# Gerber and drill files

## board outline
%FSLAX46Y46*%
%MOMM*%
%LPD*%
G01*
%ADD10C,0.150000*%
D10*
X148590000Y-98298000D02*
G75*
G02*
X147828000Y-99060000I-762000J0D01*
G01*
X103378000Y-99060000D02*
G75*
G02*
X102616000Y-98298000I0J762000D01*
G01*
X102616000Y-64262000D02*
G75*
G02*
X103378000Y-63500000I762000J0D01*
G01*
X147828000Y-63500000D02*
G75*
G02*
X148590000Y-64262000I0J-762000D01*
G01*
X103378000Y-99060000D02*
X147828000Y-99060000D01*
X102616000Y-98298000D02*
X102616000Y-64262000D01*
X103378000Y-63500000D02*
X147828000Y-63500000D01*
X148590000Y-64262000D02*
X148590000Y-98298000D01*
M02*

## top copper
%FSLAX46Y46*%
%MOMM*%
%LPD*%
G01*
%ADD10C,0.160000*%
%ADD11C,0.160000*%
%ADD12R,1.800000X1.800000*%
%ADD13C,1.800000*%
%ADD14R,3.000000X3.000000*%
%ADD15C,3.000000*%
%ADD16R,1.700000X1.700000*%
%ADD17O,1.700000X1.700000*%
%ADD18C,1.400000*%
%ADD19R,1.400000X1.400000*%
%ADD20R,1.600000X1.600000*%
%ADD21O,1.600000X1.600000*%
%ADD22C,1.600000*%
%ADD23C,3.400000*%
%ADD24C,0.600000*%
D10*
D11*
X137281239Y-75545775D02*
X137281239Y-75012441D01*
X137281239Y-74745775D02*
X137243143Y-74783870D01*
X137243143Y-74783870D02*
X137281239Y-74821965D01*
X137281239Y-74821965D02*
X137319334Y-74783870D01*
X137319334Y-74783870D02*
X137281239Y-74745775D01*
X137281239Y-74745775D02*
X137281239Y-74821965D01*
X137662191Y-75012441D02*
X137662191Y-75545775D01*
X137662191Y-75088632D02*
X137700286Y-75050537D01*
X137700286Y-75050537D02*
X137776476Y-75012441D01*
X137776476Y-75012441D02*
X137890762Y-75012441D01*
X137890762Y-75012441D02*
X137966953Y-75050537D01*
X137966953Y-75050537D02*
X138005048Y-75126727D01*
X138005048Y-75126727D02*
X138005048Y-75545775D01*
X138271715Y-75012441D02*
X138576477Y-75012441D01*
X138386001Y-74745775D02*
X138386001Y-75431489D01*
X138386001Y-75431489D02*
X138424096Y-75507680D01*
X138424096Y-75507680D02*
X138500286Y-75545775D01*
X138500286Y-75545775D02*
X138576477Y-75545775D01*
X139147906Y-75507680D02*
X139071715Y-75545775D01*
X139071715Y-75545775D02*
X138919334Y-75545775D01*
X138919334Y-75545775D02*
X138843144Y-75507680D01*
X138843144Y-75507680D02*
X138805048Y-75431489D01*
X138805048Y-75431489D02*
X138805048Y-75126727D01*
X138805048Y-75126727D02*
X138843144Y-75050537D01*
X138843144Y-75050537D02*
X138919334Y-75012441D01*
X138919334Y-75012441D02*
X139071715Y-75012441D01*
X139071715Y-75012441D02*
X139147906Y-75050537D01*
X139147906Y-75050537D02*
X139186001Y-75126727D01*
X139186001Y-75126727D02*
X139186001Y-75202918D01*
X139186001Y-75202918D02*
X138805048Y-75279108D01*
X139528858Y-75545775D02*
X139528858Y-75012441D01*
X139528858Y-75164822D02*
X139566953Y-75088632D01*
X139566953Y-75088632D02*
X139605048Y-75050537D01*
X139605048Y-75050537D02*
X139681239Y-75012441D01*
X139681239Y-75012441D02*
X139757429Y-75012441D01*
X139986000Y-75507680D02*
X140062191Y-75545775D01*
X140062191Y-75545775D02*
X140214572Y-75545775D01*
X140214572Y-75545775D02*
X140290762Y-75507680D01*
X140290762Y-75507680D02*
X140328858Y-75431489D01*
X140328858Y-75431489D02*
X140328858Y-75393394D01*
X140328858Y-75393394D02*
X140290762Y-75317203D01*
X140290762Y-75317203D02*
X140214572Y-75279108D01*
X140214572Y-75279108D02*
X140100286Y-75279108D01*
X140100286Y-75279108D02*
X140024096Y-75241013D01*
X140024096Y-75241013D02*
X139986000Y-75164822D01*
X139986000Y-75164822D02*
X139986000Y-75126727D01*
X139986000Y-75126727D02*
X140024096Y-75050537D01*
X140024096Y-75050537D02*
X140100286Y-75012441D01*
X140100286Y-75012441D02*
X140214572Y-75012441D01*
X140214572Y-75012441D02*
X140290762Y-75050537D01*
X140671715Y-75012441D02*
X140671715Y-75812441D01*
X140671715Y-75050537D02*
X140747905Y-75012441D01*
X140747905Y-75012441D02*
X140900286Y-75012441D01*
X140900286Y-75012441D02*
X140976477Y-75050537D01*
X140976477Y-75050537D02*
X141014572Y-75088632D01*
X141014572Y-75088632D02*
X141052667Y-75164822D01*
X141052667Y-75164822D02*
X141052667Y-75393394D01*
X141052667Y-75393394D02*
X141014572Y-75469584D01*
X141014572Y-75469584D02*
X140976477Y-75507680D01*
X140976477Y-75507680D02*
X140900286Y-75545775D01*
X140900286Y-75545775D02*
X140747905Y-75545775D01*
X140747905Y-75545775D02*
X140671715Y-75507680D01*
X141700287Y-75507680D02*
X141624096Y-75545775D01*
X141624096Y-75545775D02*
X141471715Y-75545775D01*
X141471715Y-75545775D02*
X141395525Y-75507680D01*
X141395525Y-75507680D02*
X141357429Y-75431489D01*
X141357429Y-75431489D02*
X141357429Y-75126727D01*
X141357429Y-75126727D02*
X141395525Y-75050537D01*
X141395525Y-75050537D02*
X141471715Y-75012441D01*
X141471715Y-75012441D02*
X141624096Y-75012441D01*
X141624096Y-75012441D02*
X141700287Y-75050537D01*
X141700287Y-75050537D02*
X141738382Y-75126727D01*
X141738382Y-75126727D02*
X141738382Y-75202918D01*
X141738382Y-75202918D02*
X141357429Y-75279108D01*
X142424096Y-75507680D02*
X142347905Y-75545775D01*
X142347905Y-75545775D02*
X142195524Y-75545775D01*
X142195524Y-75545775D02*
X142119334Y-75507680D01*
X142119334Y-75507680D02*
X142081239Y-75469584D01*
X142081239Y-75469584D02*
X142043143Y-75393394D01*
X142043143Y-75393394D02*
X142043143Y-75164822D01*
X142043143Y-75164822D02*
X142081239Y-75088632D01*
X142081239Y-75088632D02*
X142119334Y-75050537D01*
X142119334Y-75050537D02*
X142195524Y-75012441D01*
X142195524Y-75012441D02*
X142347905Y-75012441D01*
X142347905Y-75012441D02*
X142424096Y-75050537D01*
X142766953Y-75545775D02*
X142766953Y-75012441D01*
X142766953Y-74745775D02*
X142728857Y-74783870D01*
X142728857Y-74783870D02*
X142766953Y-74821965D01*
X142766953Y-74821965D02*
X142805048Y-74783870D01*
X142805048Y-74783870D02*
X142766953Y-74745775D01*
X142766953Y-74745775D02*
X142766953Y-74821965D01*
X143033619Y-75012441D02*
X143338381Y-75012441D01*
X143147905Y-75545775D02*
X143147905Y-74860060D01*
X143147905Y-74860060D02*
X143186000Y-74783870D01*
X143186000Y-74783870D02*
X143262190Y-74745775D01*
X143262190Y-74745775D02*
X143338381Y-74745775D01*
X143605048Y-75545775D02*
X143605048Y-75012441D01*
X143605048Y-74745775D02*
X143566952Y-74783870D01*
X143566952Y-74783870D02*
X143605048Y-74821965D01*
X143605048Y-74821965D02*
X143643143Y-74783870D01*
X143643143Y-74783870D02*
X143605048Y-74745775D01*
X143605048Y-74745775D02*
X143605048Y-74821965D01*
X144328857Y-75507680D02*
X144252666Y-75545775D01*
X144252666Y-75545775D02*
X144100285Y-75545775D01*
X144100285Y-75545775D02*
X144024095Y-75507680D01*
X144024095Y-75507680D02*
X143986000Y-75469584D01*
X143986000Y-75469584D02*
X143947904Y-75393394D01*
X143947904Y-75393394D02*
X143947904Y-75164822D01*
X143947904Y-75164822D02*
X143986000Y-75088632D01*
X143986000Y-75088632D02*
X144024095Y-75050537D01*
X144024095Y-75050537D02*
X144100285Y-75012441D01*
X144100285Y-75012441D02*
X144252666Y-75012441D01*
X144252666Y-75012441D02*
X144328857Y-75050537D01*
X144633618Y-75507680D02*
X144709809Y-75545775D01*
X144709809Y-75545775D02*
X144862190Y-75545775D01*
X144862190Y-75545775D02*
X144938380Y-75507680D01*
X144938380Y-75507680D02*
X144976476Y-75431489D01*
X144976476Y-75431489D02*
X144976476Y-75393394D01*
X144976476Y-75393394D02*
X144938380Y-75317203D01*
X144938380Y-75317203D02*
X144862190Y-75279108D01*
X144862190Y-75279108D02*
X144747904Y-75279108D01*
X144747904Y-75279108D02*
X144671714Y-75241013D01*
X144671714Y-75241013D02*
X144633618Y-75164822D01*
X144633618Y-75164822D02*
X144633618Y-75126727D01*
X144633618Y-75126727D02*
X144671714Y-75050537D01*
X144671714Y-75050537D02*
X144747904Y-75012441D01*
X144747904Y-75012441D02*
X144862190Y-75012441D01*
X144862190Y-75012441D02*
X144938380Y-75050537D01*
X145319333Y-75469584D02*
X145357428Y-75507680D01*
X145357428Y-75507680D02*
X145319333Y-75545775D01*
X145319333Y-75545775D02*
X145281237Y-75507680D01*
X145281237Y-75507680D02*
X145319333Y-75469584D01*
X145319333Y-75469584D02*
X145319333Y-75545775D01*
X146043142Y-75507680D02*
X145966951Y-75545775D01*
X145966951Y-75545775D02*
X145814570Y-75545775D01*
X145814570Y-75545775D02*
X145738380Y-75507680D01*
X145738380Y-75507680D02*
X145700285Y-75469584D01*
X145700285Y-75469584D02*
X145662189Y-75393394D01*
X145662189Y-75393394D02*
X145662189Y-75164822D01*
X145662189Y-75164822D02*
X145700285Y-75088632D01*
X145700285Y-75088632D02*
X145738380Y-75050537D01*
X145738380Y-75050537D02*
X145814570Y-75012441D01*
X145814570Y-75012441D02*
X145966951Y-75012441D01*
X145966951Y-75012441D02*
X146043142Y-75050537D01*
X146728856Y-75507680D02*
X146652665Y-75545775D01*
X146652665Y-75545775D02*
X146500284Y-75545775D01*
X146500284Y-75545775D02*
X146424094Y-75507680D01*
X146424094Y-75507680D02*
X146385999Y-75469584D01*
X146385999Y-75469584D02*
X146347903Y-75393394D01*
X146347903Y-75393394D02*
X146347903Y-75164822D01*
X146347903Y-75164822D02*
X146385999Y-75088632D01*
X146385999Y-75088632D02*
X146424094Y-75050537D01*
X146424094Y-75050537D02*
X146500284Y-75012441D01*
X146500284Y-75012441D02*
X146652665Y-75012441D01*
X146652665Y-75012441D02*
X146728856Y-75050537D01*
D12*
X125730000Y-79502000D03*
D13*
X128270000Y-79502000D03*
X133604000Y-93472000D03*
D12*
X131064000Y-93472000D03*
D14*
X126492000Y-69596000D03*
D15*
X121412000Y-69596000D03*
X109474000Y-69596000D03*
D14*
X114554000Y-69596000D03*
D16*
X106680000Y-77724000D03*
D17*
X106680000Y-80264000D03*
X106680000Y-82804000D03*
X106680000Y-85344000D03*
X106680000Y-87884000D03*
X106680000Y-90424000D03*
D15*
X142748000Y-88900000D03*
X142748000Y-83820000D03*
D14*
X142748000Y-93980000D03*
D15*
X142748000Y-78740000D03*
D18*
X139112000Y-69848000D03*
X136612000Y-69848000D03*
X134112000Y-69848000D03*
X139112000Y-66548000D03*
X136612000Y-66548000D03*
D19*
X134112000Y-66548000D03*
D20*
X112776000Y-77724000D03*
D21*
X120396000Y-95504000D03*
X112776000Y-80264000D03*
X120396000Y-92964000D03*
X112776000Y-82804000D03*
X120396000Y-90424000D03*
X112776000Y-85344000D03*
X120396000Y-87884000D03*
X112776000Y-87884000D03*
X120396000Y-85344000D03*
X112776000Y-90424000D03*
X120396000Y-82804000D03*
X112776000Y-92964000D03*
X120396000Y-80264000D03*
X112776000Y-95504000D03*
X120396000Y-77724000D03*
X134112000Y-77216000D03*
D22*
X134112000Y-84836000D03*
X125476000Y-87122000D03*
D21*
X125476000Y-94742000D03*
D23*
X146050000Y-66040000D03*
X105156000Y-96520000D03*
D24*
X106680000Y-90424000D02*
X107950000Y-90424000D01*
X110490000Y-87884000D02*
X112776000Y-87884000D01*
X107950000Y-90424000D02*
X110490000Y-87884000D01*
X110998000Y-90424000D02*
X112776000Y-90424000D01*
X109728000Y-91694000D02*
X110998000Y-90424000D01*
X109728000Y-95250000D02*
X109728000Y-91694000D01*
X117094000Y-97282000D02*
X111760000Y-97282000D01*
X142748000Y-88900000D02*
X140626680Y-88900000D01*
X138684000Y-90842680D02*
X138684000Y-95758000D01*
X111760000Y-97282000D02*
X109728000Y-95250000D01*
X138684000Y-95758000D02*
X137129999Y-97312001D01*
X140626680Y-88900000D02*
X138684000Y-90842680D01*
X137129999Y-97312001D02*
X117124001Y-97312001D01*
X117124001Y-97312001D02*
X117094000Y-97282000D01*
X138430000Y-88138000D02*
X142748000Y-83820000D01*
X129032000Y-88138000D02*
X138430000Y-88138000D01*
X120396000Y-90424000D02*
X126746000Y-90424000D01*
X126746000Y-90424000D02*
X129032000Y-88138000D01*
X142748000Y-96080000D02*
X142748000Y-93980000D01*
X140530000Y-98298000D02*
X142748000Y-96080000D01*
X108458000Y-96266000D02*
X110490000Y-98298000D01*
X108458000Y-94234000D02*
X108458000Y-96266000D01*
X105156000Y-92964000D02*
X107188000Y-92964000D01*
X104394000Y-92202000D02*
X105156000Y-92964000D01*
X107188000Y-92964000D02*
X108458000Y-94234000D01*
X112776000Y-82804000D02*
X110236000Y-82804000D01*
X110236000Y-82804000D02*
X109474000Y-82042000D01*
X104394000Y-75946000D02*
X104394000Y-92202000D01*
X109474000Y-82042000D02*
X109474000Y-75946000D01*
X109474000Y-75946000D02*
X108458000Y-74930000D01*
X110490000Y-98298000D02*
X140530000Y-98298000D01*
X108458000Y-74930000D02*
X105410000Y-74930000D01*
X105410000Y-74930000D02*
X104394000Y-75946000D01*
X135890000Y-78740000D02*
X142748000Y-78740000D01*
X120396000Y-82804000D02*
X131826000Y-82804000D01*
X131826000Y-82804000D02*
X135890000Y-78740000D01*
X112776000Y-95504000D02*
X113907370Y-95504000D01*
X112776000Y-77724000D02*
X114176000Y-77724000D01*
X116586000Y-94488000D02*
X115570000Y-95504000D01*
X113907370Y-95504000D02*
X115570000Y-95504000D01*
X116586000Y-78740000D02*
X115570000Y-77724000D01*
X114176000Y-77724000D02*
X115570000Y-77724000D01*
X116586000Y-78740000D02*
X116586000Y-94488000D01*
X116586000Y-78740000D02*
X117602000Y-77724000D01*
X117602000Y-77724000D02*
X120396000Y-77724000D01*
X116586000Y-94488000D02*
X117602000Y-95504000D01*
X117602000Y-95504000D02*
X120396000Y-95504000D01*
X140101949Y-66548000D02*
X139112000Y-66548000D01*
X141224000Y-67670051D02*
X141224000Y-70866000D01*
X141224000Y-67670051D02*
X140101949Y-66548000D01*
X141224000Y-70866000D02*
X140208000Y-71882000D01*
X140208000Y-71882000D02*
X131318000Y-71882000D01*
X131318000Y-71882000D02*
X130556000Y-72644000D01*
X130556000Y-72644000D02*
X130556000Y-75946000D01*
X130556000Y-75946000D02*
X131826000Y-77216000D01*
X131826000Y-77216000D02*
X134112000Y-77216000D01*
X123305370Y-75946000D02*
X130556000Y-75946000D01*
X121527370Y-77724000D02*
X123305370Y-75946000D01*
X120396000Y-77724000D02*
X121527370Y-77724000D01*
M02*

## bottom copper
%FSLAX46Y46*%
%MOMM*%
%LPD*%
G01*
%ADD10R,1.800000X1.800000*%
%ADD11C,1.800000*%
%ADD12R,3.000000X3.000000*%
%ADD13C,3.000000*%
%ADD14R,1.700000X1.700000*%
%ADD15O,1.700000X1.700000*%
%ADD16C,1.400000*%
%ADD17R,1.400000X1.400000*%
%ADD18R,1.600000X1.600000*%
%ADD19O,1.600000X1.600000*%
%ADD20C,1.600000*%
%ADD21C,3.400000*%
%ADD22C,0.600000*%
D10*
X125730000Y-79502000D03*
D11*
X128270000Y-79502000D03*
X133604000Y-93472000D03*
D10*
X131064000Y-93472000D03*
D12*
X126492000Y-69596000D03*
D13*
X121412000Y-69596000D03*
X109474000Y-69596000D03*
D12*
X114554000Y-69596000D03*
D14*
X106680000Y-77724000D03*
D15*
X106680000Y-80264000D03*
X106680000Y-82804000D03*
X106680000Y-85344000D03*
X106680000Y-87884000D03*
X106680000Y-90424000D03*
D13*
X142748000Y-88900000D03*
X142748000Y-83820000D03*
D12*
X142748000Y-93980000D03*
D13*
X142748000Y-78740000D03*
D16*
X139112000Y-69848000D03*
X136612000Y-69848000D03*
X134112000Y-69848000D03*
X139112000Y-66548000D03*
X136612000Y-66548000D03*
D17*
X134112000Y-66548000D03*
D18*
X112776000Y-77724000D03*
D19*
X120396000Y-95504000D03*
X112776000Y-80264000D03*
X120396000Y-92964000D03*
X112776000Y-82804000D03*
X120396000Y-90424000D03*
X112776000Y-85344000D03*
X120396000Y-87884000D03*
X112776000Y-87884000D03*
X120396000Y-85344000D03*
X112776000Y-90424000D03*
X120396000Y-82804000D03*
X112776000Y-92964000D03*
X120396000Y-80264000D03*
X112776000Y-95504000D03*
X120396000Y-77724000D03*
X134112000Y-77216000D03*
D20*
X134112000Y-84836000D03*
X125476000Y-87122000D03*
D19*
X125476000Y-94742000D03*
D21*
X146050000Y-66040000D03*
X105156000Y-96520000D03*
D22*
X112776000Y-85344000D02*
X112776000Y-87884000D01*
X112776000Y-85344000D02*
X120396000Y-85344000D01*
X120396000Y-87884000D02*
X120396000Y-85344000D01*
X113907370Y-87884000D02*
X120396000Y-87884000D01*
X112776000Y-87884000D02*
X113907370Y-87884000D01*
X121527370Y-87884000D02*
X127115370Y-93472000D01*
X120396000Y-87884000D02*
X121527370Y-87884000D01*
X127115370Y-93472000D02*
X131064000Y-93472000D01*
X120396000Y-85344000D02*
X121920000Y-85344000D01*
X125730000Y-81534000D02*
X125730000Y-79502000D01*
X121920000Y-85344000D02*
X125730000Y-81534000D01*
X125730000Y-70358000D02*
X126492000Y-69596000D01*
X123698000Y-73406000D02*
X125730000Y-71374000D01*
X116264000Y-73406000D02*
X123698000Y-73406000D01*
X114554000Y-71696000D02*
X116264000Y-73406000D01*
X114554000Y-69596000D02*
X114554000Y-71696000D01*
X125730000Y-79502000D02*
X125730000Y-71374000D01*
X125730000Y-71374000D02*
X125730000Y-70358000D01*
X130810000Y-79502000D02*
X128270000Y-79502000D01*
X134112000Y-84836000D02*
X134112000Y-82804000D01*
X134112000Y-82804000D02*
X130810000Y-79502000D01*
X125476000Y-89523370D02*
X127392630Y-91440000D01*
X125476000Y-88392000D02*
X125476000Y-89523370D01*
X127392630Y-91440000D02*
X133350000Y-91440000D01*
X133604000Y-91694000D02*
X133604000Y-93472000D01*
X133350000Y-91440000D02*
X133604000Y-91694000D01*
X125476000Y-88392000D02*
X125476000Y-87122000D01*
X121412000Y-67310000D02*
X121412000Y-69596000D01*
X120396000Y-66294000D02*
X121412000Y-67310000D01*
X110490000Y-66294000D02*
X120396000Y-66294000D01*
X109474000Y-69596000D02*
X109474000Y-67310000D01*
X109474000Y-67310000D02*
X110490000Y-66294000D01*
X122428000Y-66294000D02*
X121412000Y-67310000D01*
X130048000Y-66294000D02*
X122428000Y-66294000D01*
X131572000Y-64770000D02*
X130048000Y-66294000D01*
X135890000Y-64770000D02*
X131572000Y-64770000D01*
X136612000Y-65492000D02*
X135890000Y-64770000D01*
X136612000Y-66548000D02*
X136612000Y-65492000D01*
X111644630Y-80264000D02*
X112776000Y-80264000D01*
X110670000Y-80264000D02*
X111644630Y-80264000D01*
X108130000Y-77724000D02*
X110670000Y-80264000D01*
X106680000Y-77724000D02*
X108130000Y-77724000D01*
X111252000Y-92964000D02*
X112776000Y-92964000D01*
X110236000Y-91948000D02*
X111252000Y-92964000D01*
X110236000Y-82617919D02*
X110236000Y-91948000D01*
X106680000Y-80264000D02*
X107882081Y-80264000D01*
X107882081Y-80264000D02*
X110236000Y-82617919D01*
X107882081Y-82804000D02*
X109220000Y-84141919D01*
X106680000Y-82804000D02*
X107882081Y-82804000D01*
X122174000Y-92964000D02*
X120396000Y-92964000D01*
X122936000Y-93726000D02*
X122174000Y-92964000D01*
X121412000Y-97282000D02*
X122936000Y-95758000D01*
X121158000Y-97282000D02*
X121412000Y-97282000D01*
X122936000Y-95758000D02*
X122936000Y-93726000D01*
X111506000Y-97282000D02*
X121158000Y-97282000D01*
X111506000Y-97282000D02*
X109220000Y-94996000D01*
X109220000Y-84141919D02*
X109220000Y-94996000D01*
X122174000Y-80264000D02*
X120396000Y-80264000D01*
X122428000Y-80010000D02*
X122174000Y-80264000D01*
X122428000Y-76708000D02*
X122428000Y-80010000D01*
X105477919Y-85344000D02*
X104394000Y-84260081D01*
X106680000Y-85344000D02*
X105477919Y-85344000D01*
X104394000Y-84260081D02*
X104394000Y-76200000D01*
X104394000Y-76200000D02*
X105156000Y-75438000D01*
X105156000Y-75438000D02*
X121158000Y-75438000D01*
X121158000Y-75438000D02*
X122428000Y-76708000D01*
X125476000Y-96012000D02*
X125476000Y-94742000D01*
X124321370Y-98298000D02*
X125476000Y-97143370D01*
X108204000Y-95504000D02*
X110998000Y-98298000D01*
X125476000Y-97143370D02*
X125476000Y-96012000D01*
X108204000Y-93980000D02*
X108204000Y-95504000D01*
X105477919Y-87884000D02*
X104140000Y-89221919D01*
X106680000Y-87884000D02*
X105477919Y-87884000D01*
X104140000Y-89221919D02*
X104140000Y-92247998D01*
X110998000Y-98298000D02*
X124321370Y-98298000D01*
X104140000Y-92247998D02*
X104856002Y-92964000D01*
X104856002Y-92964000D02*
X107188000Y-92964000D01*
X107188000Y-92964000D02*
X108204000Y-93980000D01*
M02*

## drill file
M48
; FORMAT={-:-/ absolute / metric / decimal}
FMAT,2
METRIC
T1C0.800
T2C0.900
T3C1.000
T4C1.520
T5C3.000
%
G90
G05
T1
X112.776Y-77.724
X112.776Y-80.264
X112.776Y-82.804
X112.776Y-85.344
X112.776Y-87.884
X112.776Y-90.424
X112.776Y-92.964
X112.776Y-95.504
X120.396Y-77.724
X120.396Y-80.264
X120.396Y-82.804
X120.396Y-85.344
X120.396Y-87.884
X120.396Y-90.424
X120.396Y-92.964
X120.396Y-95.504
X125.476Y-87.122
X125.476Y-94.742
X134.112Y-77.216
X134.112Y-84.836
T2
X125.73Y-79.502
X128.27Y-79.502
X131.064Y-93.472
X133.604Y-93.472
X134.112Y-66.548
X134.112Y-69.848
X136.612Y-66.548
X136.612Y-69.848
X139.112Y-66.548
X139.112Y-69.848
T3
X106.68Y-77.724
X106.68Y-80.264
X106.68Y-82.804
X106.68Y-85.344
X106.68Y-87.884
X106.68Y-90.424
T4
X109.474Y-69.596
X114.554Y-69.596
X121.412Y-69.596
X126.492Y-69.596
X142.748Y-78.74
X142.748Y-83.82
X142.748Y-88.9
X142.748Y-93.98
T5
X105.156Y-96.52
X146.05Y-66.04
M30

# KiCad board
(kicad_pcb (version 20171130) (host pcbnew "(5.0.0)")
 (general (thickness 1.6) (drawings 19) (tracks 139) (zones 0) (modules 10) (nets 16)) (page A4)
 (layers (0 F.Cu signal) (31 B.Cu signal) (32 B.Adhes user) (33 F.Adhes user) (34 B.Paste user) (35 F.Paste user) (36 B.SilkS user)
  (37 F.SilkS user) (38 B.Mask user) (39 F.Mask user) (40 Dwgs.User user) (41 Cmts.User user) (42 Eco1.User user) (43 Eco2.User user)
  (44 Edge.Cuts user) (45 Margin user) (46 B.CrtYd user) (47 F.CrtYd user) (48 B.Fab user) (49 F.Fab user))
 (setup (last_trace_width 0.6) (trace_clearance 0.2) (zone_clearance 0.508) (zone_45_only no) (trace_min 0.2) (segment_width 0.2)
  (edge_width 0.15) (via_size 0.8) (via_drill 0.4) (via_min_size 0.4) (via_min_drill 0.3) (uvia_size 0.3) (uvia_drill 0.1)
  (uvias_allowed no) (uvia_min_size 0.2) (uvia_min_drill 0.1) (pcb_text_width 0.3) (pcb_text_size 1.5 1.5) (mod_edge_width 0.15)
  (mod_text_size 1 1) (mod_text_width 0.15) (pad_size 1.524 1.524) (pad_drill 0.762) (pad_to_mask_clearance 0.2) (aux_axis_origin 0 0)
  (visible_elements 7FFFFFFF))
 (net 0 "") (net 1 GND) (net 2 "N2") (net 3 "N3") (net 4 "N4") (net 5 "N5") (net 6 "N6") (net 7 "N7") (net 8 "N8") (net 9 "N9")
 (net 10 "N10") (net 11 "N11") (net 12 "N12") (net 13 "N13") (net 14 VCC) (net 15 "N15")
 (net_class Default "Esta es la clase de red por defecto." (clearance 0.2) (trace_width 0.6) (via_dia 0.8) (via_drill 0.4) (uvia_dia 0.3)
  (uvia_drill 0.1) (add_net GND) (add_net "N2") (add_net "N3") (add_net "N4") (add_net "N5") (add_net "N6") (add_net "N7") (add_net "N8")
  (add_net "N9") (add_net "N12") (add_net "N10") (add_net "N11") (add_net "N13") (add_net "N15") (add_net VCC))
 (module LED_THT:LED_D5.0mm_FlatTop (layer F.Cu) (at 125.73 79.502)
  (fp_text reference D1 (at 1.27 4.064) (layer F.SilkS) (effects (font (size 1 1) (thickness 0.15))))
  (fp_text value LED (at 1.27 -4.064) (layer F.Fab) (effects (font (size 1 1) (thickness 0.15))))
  (pad 1 thru_hole rect (at 0 0) (size 1.8 1.8) (drill 0.9) (layers *.Cu *.Mask) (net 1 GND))
  (pad 2 thru_hole circle (at 2.54 0) (size 1.8 1.8) (drill 0.9) (layers *.Cu *.Mask) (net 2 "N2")))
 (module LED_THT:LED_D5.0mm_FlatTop (layer F.Cu) (at 131.064 93.472)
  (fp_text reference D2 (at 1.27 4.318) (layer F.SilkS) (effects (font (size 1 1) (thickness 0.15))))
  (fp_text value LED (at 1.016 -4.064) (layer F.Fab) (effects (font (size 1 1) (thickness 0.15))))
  (pad 2 thru_hole circle (at 2.54 0) (size 1.8 1.8) (drill 0.9) (layers *.Cu *.Mask) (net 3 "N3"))
  (pad 1 thru_hole rect (at 0 0) (size 1.8 1.8) (drill 0.9) (layers *.Cu *.Mask) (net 1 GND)))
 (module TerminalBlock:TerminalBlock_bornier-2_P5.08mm (layer F.Cu) (at 126.492 69.596 180)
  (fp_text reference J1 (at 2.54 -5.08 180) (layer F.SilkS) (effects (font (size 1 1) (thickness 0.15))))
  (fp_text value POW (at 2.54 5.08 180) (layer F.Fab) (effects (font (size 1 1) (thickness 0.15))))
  (pad 1 thru_hole rect (at 0 0 180) (size 3 3) (drill 1.52) (layers *.Cu *.Mask) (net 1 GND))
  (pad 2 thru_hole circle (at 5.08 0 180) (size 3 3) (drill 1.52) (layers *.Cu *.Mask) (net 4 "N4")))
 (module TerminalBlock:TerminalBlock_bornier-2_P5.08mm (layer F.Cu) (at 114.554 69.596 180)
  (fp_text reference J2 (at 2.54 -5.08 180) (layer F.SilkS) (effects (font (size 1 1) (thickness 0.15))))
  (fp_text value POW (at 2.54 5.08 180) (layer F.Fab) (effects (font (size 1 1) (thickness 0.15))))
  (pad 2 thru_hole circle (at 5.08 0 180) (size 3 3) (drill 1.52) (layers *.Cu *.Mask) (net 4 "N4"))
  (pad 1 thru_hole rect (at 0 0 180) (size 3 3) (drill 1.52) (layers *.Cu *.Mask) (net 1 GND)))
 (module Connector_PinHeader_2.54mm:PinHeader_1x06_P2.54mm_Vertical (layer F.Cu) (at 106.68 77.724)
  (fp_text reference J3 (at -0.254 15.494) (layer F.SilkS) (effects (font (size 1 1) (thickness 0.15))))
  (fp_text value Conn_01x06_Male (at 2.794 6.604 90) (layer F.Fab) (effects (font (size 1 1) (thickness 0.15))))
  (pad 1 thru_hole rect (at 0 0) (size 1.7 1.7) (drill 1) (layers *.Cu *.Mask) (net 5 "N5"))
  (pad 2 thru_hole oval (at 0 2.54) (size 1.7 1.7) (drill 1) (layers *.Cu *.Mask) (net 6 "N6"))
  (pad 3 thru_hole oval (at 0 5.08) (size 1.7 1.7) (drill 1) (layers *.Cu *.Mask) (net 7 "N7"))
  (pad 4 thru_hole oval (at 0 7.62) (size 1.7 1.7) (drill 1) (layers *.Cu *.Mask) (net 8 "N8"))
  (pad 5 thru_hole oval (at 0 10.16) (size 1.7 1.7) (drill 1) (layers *.Cu *.Mask) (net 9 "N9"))
  (pad 6 thru_hole oval (at 0 12.7) (size 1.7 1.7) (drill 1) (layers *.Cu *.Mask) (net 1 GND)))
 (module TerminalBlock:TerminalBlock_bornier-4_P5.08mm (layer F.Cu) (at 142.748 93.98 90)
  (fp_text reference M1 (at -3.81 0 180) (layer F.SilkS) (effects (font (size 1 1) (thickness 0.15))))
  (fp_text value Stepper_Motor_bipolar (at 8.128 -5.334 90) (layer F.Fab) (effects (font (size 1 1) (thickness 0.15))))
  (pad 2 thru_hole circle (at 5.08 0 90) (size 3 3) (drill 1.52) (layers *.Cu *.Mask) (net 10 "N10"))
  (pad 3 thru_hole circle (at 10.16 0 90) (size 3 3) (drill 1.52) (layers *.Cu *.Mask) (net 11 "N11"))
  (pad 1 thru_hole rect (at 0 0 90) (size 3 3) (drill 1.52) (layers *.Cu *.Mask) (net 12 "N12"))
  (pad 4 thru_hole circle (at 15.24 0 90) (size 3 3) (drill 1.52) (layers *.Cu *.Mask) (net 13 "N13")))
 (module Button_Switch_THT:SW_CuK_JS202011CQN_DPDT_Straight (layer F.Cu) (at 134.112 66.548)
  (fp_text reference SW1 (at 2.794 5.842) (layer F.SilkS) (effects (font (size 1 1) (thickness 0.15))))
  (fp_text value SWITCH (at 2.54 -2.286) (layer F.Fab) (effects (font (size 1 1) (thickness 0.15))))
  (pad 6 thru_hole circle (at 5 3.3) (size 1.4 1.4) (drill 0.9) (layers *.Cu *.Mask))
  (pad 5 thru_hole circle (at 2.5 3.3) (size 1.4 1.4) (drill 0.9) (layers *.Cu *.Mask))
  (pad 4 thru_hole circle (at 0 3.3) (size 1.4 1.4) (drill 0.9) (layers *.Cu *.Mask))
  (pad 3 thru_hole circle (at 5 0) (size 1.4 1.4) (drill 0.9) (layers *.Cu *.Mask) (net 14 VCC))
  (pad 2 thru_hole circle (at 2.5 0) (size 1.4 1.4) (drill 0.9) (layers *.Cu *.Mask) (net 4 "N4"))
  (pad 1 thru_hole rect (at 0 0) (size 1.4 1.4) (drill 0.9) (layers *.Cu *.Mask) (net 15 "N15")))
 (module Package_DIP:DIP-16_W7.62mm (layer F.Cu) (at 112.776 77.724)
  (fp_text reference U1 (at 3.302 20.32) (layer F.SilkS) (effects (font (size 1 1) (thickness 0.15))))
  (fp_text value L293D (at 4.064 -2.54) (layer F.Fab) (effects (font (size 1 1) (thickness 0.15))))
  (pad 1 thru_hole rect (at 0 0) (size 1.6 1.6) (drill 0.8) (layers *.Cu *.Mask) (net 14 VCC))
  (pad 9 thru_hole oval (at 7.62 17.78) (size 1.6 1.6) (drill 0.8) (layers *.Cu *.Mask) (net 14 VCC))
  (pad 2 thru_hole oval (at 0 2.54) (size 1.6 1.6) (drill 0.8) (layers *.Cu *.Mask) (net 5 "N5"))
  (pad 10 thru_hole oval (at 7.62 15.24) (size 1.6 1.6) (drill 0.8) (layers *.Cu *.Mask) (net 7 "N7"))
  (pad 3 thru_hole oval (at 0 5.08) (size 1.6 1.6) (drill 0.8) (layers *.Cu *.Mask) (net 12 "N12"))
  (pad 11 thru_hole oval (at 7.62 12.7) (size 1.6 1.6) (drill 0.8) (layers *.Cu *.Mask) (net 11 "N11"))
  (pad 4 thru_hole oval (at 0 7.62) (size 1.6 1.6) (drill 0.8) (layers *.Cu *.Mask) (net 1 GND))
  (pad 12 thru_hole oval (at 7.62 10.16) (size 1.6 1.6) (drill 0.8) (layers *.Cu *.Mask) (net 1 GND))
  (pad 5 thru_hole oval (at 0 10.16) (size 1.6 1.6) (drill 0.8) (layers *.Cu *.Mask) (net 1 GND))
  (pad 13 thru_hole oval (at 7.62 7.62) (size 1.6 1.6) (drill 0.8) (layers *.Cu *.Mask) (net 1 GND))
  (pad 6 thru_hole oval (at 0 12.7) (size 1.6 1.6) (drill 0.8) (layers *.Cu *.Mask) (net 10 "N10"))
  (pad 14 thru_hole oval (at 7.62 5.08) (size 1.6 1.6) (drill 0.8) (layers *.Cu *.Mask) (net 13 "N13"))
  (pad 7 thru_hole oval (at 0 15.24) (size 1.6 1.6) (drill 0.8) (layers *.Cu *.Mask) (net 6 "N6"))
  (pad 15 thru_hole oval (at 7.62 2.54) (size 1.6 1.6) (drill 0.8) (layers *.Cu *.Mask) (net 8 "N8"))
  (pad 8 thru_hole oval (at 0 17.78) (size 1.6 1.6) (drill 0.8) (layers *.Cu *.Mask) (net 14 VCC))
  (pad 16 thru_hole oval (at 7.62 0) (size 1.6 1.6) (drill 0.8) (layers *.Cu *.Mask) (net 14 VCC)))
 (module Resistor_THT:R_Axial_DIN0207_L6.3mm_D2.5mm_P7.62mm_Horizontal (layer F.Cu) (at 134.112 84.836 90)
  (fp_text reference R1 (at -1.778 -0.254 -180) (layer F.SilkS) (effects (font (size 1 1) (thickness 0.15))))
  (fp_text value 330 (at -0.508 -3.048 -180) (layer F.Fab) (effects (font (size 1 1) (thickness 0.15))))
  (pad 2 thru_hole oval (at 7.62 0 90) (size 1.6 1.6) (drill 0.8) (layers *.Cu *.Mask) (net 14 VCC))
  (pad 1 thru_hole circle (at 0 0 90) (size 1.6 1.6) (drill 0.8) (layers *.Cu *.Mask) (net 2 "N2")))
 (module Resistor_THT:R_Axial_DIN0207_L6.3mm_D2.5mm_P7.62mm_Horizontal (layer F.Cu) (at 125.476 87.122 270)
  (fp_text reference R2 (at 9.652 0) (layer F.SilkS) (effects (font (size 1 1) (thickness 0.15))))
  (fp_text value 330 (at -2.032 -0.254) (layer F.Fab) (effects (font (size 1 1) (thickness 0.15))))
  (pad 1 thru_hole circle (at 0 0 270) (size 1.6 1.6) (drill 0.8) (layers *.Cu *.Mask) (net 3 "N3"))
  (pad 2 thru_hole oval (at 7.62 0 270) (size 1.6 1.6) (drill 0.8) (layers *.Cu *.Mask) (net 9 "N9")))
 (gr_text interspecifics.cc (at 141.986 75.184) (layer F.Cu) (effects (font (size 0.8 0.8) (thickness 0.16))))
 (gr_arc (start 147.828 98.298) (end 147.828 99.06) (angle -90) (layer Edge.Cuts) (width 0.15))
 (gr_arc (start 103.378 98.298) (end 102.616 98.298) (angle -90) (layer Edge.Cuts) (width 0.15))
 (gr_arc (start 103.378 64.262) (end 103.378 63.5) (angle -90) (layer Edge.Cuts) (width 0.15))
 (gr_arc (start 147.828 64.262) (end 148.59 64.262) (angle -90) (layer Edge.Cuts) (width 0.15))
 (gr_line (start 103.378 99.06) (end 147.828 99.06) (layer Edge.Cuts) (width 0.15))
 (gr_line (start 102.616 98.298) (end 102.616 64.262) (layer Edge.Cuts) (width 0.15))
 (gr_line (start 103.378 63.5) (end 147.828 63.5) (layer Edge.Cuts) (width 0.15))
 (gr_line (start 148.59 64.262) (end 148.59 98.298) (layer Edge.Cuts) (width 0.15))
 (via (at 146.05 66.04) (size 3.4) (drill 3) (layers F.Cu B.Cu) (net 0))
 (via (at 105.156 96.52) (size 3.4) (drill 3) (layers F.Cu B.Cu) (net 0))
 (segment (start 112.776 85.344) (end 112.776 87.884) (width 0.6) (layer B.Cu) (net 1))
 (segment (start 112.776 85.344) (end 120.396 85.344) (width 0.6) (layer B.Cu) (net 1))
 (segment (start 120.396 87.884) (end 120.396 85.344) (width 0.6) (layer B.Cu) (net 1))
 (segment (start 113.90737 87.884) (end 120.396 87.884) (width 0.6) (layer B.Cu) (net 1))
 (segment (start 112.776 87.884) (end 113.90737 87.884) (width 0.6) (layer B.Cu) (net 1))
 (segment (start 121.52737 87.884) (end 127.11537 93.472) (width 0.6) (layer B.Cu) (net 1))
 (segment (start 120.396 87.884) (end 121.52737 87.884) (width 0.6) (layer B.Cu) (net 1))
 (segment (start 127.11537 93.472) (end 131.064 93.472) (width 0.6) (layer B.Cu) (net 1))
 (segment (start 120.396 85.344) (end 121.92 85.344) (width 0.6) (layer B.Cu) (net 1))
 (segment (start 125.73 81.534) (end 125.73 79.502) (width 0.6) (layer B.Cu) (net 1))
 (segment (start 121.92 85.344) (end 125.73 81.534) (width 0.6) (layer B.Cu) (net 1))
 (segment (start 125.73 70.358) (end 126.492 69.596) (width 0.6) (layer B.Cu) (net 1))
 (segment (start 123.698 73.406) (end 125.73 71.374) (width 0.6) (layer B.Cu) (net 1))
 (segment (start 116.264 73.406) (end 123.698 73.406) (width 0.6) (layer B.Cu) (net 1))
 (segment (start 114.554 71.696) (end 116.264 73.406) (width 0.6) (layer B.Cu) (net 1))
 (segment (start 114.554 69.596) (end 114.554 71.696) (width 0.6) (layer B.Cu) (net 1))
 (segment (start 125.73 79.502) (end 125.73 71.374) (width 0.6) (layer B.Cu) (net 1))
 (segment (start 125.73 71.374) (end 125.73 70.358) (width 0.6) (layer B.Cu) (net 1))
 (segment (start 106.68 90.424) (end 107.95 90.424) (width 0.6) (layer F.Cu) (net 1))
 (segment (start 110.49 87.884) (end 112.776 87.884) (width 0.6) (layer F.Cu) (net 1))
 (segment (start 107.95 90.424) (end 110.49 87.884) (width 0.6) (layer F.Cu) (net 1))
 (segment (start 130.81 79.502) (end 128.27 79.502) (width 0.6) (layer B.Cu) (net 2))
 (segment (start 134.112 84.836) (end 134.112 82.804) (width 0.6) (layer B.Cu) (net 2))
 (segment (start 134.112 82.804) (end 130.81 79.502) (width 0.6) (layer B.Cu) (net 2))
 (segment (start 125.476 89.52337) (end 127.39263 91.44) (width 0.6) (layer B.Cu) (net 3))
 (segment (start 125.476 88.392) (end 125.476 89.52337) (width 0.6) (layer B.Cu) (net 3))
 (segment (start 127.39263 91.44) (end 133.35 91.44) (width 0.6) (layer B.Cu) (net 3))
 (segment (start 133.604 91.694) (end 133.604 93.472) (width 0.6) (layer B.Cu) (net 3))
 (segment (start 133.35 91.44) (end 133.604 91.694) (width 0.6) (layer B.Cu) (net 3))
 (segment (start 125.476 88.392) (end 125.476 87.122) (width 0.6) (layer B.Cu) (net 3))
 (segment (start 121.412 67.31) (end 121.412 69.596) (width 0.6) (layer B.Cu) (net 4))
 (segment (start 120.396 66.294) (end 121.412 67.31) (width 0.6) (layer B.Cu) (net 4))
 (segment (start 110.49 66.294) (end 120.396 66.294) (width 0.6) (layer B.Cu) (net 4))
 (segment (start 109.474 69.596) (end 109.474 67.31) (width 0.6) (layer B.Cu) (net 4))
 (segment (start 109.474 67.31) (end 110.49 66.294) (width 0.6) (layer B.Cu) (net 4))
 (segment (start 122.428 66.294) (end 121.412 67.31) (width 0.6) (layer B.Cu) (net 4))
 (segment (start 130.048 66.294) (end 122.428 66.294) (width 0.6) (layer B.Cu) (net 4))
 (segment (start 131.572 64.77) (end 130.048 66.294) (width 0.6) (layer B.Cu) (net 4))
 (segment (start 135.89 64.77) (end 131.572 64.77) (width 0.6) (layer B.Cu) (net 4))
 (segment (start 136.612 65.492) (end 135.89 64.77) (width 0.6) (layer B.Cu) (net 4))
 (segment (start 136.612 66.548) (end 136.612 65.492) (width 0.6) (layer B.Cu) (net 4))
 (segment (start 111.64463 80.264) (end 112.776 80.264) (width 0.6) (layer B.Cu) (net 5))
 (segment (start 110.67 80.264) (end 111.64463 80.264) (width 0.6) (layer B.Cu) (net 5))
 (segment (start 108.13 77.724) (end 110.67 80.264) (width 0.6) (layer B.Cu) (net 5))
 (segment (start 106.68 77.724) (end 108.13 77.724) (width 0.6) (layer B.Cu) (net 5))
 (segment (start 111.252 92.964) (end 112.776 92.964) (width 0.6) (layer B.Cu) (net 6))
 (segment (start 110.236 91.948) (end 111.252 92.964) (width 0.6) (layer B.Cu) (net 6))
 (segment (start 110.236 82.617919) (end 110.236 91.948) (width 0.6) (layer B.Cu) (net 6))
 (segment (start 106.68 80.264) (end 107.882081 80.264) (width 0.6) (layer B.Cu) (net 6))
 (segment (start 107.882081 80.264) (end 110.236 82.617919) (width 0.6) (layer B.Cu) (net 6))
 (segment (start 107.882081 82.804) (end 109.22 84.141919) (width 0.6) (layer B.Cu) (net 7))
 (segment (start 106.68 82.804) (end 107.882081 82.804) (width 0.6) (layer B.Cu) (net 7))
 (segment (start 122.174 92.964) (end 120.396 92.964) (width 0.6) (layer B.Cu) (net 7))
 (segment (start 122.936 93.726) (end 122.174 92.964) (width 0.6) (layer B.Cu) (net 7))
 (segment (start 121.412 97.282) (end 122.936 95.758) (width 0.6) (layer B.Cu) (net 7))
 (segment (start 121.158 97.282) (end 121.412 97.282) (width 0.6) (layer B.Cu) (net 7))
 (segment (start 122.936 95.758) (end 122.936 93.726) (width 0.6) (layer B.Cu) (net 7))
 (segment (start 111.506 97.282) (end 121.158 97.282) (width 0.6) (layer B.Cu) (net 7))
 (segment (start 111.506 97.282) (end 109.22 94.996) (width 0.6) (layer B.Cu) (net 7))
 (segment (start 109.22 84.141919) (end 109.22 94.996) (width 0.6) (layer B.Cu) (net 7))
 (segment (start 122.174 80.264) (end 120.396 80.264) (width 0.6) (layer B.Cu) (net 8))
 (segment (start 122.428 80.01) (end 122.174 80.264) (width 0.6) (layer B.Cu) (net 8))
 (segment (start 122.428 76.708) (end 122.428 80.01) (width 0.6) (layer B.Cu) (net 8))
 (segment (start 105.477919 85.344) (end 104.394 84.260081) (width 0.6) (layer B.Cu) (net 8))
 (segment (start 106.68 85.344) (end 105.477919 85.344) (width 0.6) (layer B.Cu) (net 8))
 (segment (start 104.394 84.260081) (end 104.394 76.2) (width 0.6) (layer B.Cu) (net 8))
 (segment (start 104.394 76.2) (end 105.156 75.438) (width 0.6) (layer B.Cu) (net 8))
 (segment (start 105.156 75.438) (end 121.158 75.438) (width 0.6) (layer B.Cu) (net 8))
 (segment (start 121.158 75.438) (end 122.428 76.708) (width 0.6) (layer B.Cu) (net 8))
 (segment (start 125.476 96.012) (end 125.476 94.742) (width 0.6) (layer B.Cu) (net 9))
 (segment (start 124.32137 98.298) (end 125.476 97.14337) (width 0.6) (layer B.Cu) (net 9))
 (segment (start 108.204 95.504) (end 110.998 98.298) (width 0.6) (layer B.Cu) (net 9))
 (segment (start 125.476 97.14337) (end 125.476 96.012) (width 0.6) (layer B.Cu) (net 9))
 (segment (start 108.204 93.98) (end 108.204 95.504) (width 0.6) (layer B.Cu) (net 9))
 (segment (start 105.477919 87.884) (end 104.14 89.221919) (width 0.6) (layer B.Cu) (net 9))
 (segment (start 106.68 87.884) (end 105.477919 87.884) (width 0.6) (layer B.Cu) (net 9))
 (segment (start 104.14 89.221919) (end 104.14 92.247998) (width 0.6) (layer B.Cu) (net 9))
 (segment (start 110.998 98.298) (end 124.32137 98.298) (width 0.6) (layer B.Cu) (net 9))
 (segment (start 104.14 92.247998) (end 104.856002 92.964) (width 0.6) (layer B.Cu) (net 9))
 (segment (start 104.856002 92.964) (end 107.188 92.964) (width 0.6) (layer B.Cu) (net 9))
 (segment (start 107.188 92.964) (end 108.204 93.98) (width 0.6) (layer B.Cu) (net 9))
 (segment (start 110.998 90.424) (end 112.776 90.424) (width 0.6) (layer F.Cu) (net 10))
 (segment (start 109.728 91.694) (end 110.998 90.424) (width 0.6) (layer F.Cu) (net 10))
 (segment (start 109.728 95.25) (end 109.728 91.694) (width 0.6) (layer F.Cu) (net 10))
 (segment (start 117.094 97.282) (end 111.76 97.282) (width 0.6) (layer F.Cu) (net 10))
 (segment (start 142.748 88.9) (end 140.62668 88.9) (width 0.6) (layer F.Cu) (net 10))
 (segment (start 138.684 90.84268) (end 138.684 95.758) (width 0.6) (layer F.Cu) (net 10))
 (segment (start 111.76 97.282) (end 109.728 95.25) (width 0.6) (layer F.Cu) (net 10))
 (segment (start 138.684 95.758) (end 137.129999 97.312001) (width 0.6) (layer F.Cu) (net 10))
 (segment (start 140.62668 88.9) (end 138.684 90.84268) (width 0.6) (layer F.Cu) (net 10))
 (segment (start 137.129999 97.312001) (end 117.124001 97.312001) (width 0.6) (layer F.Cu) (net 10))
 (segment (start 117.124001 97.312001) (end 117.094 97.282) (width 0.6) (layer F.Cu) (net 10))
 (segment (start 138.43 88.138) (end 142.748 83.82) (width 0.6) (layer F.Cu) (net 11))
 (segment (start 129.032 88.138) (end 138.43 88.138) (width 0.6) (layer F.Cu) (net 11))
 (segment (start 120.396 90.424) (end 126.746 90.424) (width 0.6) (layer F.Cu) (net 11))
 (segment (start 126.746 90.424) (end 129.032 88.138) (width 0.6) (layer F.Cu) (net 11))
 (segment (start 142.748 96.08) (end 142.748 93.98) (width 0.6) (layer F.Cu) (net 12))
 (segment (start 140.53 98.298) (end 142.748 96.08) (width 0.6) (layer F.Cu) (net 12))
 (segment (start 108.458 96.266) (end 110.49 98.298) (width 0.6) (layer F.Cu) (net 12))
 (segment (start 108.458 94.234) (end 108.458 96.266) (width 0.6) (layer F.Cu) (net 12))
 (segment (start 105.156 92.964) (end 107.188 92.964) (width 0.6) (layer F.Cu) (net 12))
 (segment (start 104.394 92.202) (end 105.156 92.964) (width 0.6) (layer F.Cu) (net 12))
 (segment (start 107.188 92.964) (end 108.458 94.234) (width 0.6) (layer F.Cu) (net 12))
 (segment (start 112.776 82.804) (end 110.236 82.804) (width 0.6) (layer F.Cu) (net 12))
 (segment (start 110.236 82.804) (end 109.474 82.042) (width 0.6) (layer F.Cu) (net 12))
 (segment (start 104.394 75.946) (end 104.394 92.202) (width 0.6) (layer F.Cu) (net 12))
 (segment (start 109.474 82.042) (end 109.474 75.946) (width 0.6) (layer F.Cu) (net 12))
 (segment (start 109.474 75.946) (end 108.458 74.93) (width 0.6) (layer F.Cu) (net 12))
 (segment (start 110.49 98.298) (end 140.53 98.298) (width 0.6) (layer F.Cu) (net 12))
 (segment (start 108.458 74.93) (end 105.41 74.93) (width 0.6) (layer F.Cu) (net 12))
 (segment (start 105.41 74.93) (end 104.394 75.946) (width 0.6) (layer F.Cu) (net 12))
 (segment (start 135.89 78.74) (end 142.748 78.74) (width 0.6) (layer F.Cu) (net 13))
 (segment (start 120.396 82.804) (end 131.826 82.804) (width 0.6) (layer F.Cu) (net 13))
 (segment (start 131.826 82.804) (end 135.89 78.74) (width 0.6) (layer F.Cu) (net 13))
 (segment (start 112.776 95.504) (end 113.90737 95.504) (width 0.6) (layer F.Cu) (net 14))
 (segment (start 112.776 77.724) (end 114.176 77.724) (width 0.6) (layer F.Cu) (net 14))
 (segment (start 116.586 94.488) (end 115.57 95.504) (width 0.6) (layer F.Cu) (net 14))
 (segment (start 113.90737 95.504) (end 115.57 95.504) (width 0.6) (layer F.Cu) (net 14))
 (segment (start 116.586 78.74) (end 115.57 77.724) (width 0.6) (layer F.Cu) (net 14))
 (segment (start 114.176 77.724) (end 115.57 77.724) (width 0.6) (layer F.Cu) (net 14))
 (segment (start 116.586 78.74) (end 116.586 94.488) (width 0.6) (layer F.Cu) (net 14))
 (segment (start 116.586 78.74) (end 117.602 77.724) (width 0.6) (layer F.Cu) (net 14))
 (segment (start 117.602 77.724) (end 120.396 77.724) (width 0.6) (layer F.Cu) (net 14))
 (segment (start 116.586 94.488) (end 117.602 95.504) (width 0.6) (layer F.Cu) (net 14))
 (segment (start 117.602 95.504) (end 120.396 95.504) (width 0.6) (layer F.Cu) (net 14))
 (segment (start 140.101949 66.548) (end 139.112 66.548) (width 0.6) (layer F.Cu) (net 14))
 (segment (start 141.224 67.670051) (end 141.224 70.866) (width 0.6) (layer F.Cu) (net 14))
 (segment (start 141.224 67.670051) (end 140.101949 66.548) (width 0.6) (layer F.Cu) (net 14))
 (segment (start 141.224 70.866) (end 140.208 71.882) (width 0.6) (layer F.Cu) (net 14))
 (segment (start 140.208 71.882) (end 131.318 71.882) (width 0.6) (layer F.Cu) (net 14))
 (segment (start 131.318 71.882) (end 130.556 72.644) (width 0.6) (layer F.Cu) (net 14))
 (segment (start 130.556 72.644) (end 130.556 75.946) (width 0.6) (layer F.Cu) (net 14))
 (segment (start 130.556 75.946) (end 131.826 77.216) (width 0.6) (layer F.Cu) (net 14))
 (segment (start 131.826 77.216) (end 134.112 77.216) (width 0.6) (layer F.Cu) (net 14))
 (segment (start 123.30537 75.946) (end 130.556 75.946) (width 0.6) (layer F.Cu) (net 14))
 (segment (start 121.52737 77.724) (end 123.30537 75.946) (width 0.6) (layer F.Cu) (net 14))
 (segment (start 120.396 77.724) (end 121.52737 77.724) (width 0.6) (layer F.Cu) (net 14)))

